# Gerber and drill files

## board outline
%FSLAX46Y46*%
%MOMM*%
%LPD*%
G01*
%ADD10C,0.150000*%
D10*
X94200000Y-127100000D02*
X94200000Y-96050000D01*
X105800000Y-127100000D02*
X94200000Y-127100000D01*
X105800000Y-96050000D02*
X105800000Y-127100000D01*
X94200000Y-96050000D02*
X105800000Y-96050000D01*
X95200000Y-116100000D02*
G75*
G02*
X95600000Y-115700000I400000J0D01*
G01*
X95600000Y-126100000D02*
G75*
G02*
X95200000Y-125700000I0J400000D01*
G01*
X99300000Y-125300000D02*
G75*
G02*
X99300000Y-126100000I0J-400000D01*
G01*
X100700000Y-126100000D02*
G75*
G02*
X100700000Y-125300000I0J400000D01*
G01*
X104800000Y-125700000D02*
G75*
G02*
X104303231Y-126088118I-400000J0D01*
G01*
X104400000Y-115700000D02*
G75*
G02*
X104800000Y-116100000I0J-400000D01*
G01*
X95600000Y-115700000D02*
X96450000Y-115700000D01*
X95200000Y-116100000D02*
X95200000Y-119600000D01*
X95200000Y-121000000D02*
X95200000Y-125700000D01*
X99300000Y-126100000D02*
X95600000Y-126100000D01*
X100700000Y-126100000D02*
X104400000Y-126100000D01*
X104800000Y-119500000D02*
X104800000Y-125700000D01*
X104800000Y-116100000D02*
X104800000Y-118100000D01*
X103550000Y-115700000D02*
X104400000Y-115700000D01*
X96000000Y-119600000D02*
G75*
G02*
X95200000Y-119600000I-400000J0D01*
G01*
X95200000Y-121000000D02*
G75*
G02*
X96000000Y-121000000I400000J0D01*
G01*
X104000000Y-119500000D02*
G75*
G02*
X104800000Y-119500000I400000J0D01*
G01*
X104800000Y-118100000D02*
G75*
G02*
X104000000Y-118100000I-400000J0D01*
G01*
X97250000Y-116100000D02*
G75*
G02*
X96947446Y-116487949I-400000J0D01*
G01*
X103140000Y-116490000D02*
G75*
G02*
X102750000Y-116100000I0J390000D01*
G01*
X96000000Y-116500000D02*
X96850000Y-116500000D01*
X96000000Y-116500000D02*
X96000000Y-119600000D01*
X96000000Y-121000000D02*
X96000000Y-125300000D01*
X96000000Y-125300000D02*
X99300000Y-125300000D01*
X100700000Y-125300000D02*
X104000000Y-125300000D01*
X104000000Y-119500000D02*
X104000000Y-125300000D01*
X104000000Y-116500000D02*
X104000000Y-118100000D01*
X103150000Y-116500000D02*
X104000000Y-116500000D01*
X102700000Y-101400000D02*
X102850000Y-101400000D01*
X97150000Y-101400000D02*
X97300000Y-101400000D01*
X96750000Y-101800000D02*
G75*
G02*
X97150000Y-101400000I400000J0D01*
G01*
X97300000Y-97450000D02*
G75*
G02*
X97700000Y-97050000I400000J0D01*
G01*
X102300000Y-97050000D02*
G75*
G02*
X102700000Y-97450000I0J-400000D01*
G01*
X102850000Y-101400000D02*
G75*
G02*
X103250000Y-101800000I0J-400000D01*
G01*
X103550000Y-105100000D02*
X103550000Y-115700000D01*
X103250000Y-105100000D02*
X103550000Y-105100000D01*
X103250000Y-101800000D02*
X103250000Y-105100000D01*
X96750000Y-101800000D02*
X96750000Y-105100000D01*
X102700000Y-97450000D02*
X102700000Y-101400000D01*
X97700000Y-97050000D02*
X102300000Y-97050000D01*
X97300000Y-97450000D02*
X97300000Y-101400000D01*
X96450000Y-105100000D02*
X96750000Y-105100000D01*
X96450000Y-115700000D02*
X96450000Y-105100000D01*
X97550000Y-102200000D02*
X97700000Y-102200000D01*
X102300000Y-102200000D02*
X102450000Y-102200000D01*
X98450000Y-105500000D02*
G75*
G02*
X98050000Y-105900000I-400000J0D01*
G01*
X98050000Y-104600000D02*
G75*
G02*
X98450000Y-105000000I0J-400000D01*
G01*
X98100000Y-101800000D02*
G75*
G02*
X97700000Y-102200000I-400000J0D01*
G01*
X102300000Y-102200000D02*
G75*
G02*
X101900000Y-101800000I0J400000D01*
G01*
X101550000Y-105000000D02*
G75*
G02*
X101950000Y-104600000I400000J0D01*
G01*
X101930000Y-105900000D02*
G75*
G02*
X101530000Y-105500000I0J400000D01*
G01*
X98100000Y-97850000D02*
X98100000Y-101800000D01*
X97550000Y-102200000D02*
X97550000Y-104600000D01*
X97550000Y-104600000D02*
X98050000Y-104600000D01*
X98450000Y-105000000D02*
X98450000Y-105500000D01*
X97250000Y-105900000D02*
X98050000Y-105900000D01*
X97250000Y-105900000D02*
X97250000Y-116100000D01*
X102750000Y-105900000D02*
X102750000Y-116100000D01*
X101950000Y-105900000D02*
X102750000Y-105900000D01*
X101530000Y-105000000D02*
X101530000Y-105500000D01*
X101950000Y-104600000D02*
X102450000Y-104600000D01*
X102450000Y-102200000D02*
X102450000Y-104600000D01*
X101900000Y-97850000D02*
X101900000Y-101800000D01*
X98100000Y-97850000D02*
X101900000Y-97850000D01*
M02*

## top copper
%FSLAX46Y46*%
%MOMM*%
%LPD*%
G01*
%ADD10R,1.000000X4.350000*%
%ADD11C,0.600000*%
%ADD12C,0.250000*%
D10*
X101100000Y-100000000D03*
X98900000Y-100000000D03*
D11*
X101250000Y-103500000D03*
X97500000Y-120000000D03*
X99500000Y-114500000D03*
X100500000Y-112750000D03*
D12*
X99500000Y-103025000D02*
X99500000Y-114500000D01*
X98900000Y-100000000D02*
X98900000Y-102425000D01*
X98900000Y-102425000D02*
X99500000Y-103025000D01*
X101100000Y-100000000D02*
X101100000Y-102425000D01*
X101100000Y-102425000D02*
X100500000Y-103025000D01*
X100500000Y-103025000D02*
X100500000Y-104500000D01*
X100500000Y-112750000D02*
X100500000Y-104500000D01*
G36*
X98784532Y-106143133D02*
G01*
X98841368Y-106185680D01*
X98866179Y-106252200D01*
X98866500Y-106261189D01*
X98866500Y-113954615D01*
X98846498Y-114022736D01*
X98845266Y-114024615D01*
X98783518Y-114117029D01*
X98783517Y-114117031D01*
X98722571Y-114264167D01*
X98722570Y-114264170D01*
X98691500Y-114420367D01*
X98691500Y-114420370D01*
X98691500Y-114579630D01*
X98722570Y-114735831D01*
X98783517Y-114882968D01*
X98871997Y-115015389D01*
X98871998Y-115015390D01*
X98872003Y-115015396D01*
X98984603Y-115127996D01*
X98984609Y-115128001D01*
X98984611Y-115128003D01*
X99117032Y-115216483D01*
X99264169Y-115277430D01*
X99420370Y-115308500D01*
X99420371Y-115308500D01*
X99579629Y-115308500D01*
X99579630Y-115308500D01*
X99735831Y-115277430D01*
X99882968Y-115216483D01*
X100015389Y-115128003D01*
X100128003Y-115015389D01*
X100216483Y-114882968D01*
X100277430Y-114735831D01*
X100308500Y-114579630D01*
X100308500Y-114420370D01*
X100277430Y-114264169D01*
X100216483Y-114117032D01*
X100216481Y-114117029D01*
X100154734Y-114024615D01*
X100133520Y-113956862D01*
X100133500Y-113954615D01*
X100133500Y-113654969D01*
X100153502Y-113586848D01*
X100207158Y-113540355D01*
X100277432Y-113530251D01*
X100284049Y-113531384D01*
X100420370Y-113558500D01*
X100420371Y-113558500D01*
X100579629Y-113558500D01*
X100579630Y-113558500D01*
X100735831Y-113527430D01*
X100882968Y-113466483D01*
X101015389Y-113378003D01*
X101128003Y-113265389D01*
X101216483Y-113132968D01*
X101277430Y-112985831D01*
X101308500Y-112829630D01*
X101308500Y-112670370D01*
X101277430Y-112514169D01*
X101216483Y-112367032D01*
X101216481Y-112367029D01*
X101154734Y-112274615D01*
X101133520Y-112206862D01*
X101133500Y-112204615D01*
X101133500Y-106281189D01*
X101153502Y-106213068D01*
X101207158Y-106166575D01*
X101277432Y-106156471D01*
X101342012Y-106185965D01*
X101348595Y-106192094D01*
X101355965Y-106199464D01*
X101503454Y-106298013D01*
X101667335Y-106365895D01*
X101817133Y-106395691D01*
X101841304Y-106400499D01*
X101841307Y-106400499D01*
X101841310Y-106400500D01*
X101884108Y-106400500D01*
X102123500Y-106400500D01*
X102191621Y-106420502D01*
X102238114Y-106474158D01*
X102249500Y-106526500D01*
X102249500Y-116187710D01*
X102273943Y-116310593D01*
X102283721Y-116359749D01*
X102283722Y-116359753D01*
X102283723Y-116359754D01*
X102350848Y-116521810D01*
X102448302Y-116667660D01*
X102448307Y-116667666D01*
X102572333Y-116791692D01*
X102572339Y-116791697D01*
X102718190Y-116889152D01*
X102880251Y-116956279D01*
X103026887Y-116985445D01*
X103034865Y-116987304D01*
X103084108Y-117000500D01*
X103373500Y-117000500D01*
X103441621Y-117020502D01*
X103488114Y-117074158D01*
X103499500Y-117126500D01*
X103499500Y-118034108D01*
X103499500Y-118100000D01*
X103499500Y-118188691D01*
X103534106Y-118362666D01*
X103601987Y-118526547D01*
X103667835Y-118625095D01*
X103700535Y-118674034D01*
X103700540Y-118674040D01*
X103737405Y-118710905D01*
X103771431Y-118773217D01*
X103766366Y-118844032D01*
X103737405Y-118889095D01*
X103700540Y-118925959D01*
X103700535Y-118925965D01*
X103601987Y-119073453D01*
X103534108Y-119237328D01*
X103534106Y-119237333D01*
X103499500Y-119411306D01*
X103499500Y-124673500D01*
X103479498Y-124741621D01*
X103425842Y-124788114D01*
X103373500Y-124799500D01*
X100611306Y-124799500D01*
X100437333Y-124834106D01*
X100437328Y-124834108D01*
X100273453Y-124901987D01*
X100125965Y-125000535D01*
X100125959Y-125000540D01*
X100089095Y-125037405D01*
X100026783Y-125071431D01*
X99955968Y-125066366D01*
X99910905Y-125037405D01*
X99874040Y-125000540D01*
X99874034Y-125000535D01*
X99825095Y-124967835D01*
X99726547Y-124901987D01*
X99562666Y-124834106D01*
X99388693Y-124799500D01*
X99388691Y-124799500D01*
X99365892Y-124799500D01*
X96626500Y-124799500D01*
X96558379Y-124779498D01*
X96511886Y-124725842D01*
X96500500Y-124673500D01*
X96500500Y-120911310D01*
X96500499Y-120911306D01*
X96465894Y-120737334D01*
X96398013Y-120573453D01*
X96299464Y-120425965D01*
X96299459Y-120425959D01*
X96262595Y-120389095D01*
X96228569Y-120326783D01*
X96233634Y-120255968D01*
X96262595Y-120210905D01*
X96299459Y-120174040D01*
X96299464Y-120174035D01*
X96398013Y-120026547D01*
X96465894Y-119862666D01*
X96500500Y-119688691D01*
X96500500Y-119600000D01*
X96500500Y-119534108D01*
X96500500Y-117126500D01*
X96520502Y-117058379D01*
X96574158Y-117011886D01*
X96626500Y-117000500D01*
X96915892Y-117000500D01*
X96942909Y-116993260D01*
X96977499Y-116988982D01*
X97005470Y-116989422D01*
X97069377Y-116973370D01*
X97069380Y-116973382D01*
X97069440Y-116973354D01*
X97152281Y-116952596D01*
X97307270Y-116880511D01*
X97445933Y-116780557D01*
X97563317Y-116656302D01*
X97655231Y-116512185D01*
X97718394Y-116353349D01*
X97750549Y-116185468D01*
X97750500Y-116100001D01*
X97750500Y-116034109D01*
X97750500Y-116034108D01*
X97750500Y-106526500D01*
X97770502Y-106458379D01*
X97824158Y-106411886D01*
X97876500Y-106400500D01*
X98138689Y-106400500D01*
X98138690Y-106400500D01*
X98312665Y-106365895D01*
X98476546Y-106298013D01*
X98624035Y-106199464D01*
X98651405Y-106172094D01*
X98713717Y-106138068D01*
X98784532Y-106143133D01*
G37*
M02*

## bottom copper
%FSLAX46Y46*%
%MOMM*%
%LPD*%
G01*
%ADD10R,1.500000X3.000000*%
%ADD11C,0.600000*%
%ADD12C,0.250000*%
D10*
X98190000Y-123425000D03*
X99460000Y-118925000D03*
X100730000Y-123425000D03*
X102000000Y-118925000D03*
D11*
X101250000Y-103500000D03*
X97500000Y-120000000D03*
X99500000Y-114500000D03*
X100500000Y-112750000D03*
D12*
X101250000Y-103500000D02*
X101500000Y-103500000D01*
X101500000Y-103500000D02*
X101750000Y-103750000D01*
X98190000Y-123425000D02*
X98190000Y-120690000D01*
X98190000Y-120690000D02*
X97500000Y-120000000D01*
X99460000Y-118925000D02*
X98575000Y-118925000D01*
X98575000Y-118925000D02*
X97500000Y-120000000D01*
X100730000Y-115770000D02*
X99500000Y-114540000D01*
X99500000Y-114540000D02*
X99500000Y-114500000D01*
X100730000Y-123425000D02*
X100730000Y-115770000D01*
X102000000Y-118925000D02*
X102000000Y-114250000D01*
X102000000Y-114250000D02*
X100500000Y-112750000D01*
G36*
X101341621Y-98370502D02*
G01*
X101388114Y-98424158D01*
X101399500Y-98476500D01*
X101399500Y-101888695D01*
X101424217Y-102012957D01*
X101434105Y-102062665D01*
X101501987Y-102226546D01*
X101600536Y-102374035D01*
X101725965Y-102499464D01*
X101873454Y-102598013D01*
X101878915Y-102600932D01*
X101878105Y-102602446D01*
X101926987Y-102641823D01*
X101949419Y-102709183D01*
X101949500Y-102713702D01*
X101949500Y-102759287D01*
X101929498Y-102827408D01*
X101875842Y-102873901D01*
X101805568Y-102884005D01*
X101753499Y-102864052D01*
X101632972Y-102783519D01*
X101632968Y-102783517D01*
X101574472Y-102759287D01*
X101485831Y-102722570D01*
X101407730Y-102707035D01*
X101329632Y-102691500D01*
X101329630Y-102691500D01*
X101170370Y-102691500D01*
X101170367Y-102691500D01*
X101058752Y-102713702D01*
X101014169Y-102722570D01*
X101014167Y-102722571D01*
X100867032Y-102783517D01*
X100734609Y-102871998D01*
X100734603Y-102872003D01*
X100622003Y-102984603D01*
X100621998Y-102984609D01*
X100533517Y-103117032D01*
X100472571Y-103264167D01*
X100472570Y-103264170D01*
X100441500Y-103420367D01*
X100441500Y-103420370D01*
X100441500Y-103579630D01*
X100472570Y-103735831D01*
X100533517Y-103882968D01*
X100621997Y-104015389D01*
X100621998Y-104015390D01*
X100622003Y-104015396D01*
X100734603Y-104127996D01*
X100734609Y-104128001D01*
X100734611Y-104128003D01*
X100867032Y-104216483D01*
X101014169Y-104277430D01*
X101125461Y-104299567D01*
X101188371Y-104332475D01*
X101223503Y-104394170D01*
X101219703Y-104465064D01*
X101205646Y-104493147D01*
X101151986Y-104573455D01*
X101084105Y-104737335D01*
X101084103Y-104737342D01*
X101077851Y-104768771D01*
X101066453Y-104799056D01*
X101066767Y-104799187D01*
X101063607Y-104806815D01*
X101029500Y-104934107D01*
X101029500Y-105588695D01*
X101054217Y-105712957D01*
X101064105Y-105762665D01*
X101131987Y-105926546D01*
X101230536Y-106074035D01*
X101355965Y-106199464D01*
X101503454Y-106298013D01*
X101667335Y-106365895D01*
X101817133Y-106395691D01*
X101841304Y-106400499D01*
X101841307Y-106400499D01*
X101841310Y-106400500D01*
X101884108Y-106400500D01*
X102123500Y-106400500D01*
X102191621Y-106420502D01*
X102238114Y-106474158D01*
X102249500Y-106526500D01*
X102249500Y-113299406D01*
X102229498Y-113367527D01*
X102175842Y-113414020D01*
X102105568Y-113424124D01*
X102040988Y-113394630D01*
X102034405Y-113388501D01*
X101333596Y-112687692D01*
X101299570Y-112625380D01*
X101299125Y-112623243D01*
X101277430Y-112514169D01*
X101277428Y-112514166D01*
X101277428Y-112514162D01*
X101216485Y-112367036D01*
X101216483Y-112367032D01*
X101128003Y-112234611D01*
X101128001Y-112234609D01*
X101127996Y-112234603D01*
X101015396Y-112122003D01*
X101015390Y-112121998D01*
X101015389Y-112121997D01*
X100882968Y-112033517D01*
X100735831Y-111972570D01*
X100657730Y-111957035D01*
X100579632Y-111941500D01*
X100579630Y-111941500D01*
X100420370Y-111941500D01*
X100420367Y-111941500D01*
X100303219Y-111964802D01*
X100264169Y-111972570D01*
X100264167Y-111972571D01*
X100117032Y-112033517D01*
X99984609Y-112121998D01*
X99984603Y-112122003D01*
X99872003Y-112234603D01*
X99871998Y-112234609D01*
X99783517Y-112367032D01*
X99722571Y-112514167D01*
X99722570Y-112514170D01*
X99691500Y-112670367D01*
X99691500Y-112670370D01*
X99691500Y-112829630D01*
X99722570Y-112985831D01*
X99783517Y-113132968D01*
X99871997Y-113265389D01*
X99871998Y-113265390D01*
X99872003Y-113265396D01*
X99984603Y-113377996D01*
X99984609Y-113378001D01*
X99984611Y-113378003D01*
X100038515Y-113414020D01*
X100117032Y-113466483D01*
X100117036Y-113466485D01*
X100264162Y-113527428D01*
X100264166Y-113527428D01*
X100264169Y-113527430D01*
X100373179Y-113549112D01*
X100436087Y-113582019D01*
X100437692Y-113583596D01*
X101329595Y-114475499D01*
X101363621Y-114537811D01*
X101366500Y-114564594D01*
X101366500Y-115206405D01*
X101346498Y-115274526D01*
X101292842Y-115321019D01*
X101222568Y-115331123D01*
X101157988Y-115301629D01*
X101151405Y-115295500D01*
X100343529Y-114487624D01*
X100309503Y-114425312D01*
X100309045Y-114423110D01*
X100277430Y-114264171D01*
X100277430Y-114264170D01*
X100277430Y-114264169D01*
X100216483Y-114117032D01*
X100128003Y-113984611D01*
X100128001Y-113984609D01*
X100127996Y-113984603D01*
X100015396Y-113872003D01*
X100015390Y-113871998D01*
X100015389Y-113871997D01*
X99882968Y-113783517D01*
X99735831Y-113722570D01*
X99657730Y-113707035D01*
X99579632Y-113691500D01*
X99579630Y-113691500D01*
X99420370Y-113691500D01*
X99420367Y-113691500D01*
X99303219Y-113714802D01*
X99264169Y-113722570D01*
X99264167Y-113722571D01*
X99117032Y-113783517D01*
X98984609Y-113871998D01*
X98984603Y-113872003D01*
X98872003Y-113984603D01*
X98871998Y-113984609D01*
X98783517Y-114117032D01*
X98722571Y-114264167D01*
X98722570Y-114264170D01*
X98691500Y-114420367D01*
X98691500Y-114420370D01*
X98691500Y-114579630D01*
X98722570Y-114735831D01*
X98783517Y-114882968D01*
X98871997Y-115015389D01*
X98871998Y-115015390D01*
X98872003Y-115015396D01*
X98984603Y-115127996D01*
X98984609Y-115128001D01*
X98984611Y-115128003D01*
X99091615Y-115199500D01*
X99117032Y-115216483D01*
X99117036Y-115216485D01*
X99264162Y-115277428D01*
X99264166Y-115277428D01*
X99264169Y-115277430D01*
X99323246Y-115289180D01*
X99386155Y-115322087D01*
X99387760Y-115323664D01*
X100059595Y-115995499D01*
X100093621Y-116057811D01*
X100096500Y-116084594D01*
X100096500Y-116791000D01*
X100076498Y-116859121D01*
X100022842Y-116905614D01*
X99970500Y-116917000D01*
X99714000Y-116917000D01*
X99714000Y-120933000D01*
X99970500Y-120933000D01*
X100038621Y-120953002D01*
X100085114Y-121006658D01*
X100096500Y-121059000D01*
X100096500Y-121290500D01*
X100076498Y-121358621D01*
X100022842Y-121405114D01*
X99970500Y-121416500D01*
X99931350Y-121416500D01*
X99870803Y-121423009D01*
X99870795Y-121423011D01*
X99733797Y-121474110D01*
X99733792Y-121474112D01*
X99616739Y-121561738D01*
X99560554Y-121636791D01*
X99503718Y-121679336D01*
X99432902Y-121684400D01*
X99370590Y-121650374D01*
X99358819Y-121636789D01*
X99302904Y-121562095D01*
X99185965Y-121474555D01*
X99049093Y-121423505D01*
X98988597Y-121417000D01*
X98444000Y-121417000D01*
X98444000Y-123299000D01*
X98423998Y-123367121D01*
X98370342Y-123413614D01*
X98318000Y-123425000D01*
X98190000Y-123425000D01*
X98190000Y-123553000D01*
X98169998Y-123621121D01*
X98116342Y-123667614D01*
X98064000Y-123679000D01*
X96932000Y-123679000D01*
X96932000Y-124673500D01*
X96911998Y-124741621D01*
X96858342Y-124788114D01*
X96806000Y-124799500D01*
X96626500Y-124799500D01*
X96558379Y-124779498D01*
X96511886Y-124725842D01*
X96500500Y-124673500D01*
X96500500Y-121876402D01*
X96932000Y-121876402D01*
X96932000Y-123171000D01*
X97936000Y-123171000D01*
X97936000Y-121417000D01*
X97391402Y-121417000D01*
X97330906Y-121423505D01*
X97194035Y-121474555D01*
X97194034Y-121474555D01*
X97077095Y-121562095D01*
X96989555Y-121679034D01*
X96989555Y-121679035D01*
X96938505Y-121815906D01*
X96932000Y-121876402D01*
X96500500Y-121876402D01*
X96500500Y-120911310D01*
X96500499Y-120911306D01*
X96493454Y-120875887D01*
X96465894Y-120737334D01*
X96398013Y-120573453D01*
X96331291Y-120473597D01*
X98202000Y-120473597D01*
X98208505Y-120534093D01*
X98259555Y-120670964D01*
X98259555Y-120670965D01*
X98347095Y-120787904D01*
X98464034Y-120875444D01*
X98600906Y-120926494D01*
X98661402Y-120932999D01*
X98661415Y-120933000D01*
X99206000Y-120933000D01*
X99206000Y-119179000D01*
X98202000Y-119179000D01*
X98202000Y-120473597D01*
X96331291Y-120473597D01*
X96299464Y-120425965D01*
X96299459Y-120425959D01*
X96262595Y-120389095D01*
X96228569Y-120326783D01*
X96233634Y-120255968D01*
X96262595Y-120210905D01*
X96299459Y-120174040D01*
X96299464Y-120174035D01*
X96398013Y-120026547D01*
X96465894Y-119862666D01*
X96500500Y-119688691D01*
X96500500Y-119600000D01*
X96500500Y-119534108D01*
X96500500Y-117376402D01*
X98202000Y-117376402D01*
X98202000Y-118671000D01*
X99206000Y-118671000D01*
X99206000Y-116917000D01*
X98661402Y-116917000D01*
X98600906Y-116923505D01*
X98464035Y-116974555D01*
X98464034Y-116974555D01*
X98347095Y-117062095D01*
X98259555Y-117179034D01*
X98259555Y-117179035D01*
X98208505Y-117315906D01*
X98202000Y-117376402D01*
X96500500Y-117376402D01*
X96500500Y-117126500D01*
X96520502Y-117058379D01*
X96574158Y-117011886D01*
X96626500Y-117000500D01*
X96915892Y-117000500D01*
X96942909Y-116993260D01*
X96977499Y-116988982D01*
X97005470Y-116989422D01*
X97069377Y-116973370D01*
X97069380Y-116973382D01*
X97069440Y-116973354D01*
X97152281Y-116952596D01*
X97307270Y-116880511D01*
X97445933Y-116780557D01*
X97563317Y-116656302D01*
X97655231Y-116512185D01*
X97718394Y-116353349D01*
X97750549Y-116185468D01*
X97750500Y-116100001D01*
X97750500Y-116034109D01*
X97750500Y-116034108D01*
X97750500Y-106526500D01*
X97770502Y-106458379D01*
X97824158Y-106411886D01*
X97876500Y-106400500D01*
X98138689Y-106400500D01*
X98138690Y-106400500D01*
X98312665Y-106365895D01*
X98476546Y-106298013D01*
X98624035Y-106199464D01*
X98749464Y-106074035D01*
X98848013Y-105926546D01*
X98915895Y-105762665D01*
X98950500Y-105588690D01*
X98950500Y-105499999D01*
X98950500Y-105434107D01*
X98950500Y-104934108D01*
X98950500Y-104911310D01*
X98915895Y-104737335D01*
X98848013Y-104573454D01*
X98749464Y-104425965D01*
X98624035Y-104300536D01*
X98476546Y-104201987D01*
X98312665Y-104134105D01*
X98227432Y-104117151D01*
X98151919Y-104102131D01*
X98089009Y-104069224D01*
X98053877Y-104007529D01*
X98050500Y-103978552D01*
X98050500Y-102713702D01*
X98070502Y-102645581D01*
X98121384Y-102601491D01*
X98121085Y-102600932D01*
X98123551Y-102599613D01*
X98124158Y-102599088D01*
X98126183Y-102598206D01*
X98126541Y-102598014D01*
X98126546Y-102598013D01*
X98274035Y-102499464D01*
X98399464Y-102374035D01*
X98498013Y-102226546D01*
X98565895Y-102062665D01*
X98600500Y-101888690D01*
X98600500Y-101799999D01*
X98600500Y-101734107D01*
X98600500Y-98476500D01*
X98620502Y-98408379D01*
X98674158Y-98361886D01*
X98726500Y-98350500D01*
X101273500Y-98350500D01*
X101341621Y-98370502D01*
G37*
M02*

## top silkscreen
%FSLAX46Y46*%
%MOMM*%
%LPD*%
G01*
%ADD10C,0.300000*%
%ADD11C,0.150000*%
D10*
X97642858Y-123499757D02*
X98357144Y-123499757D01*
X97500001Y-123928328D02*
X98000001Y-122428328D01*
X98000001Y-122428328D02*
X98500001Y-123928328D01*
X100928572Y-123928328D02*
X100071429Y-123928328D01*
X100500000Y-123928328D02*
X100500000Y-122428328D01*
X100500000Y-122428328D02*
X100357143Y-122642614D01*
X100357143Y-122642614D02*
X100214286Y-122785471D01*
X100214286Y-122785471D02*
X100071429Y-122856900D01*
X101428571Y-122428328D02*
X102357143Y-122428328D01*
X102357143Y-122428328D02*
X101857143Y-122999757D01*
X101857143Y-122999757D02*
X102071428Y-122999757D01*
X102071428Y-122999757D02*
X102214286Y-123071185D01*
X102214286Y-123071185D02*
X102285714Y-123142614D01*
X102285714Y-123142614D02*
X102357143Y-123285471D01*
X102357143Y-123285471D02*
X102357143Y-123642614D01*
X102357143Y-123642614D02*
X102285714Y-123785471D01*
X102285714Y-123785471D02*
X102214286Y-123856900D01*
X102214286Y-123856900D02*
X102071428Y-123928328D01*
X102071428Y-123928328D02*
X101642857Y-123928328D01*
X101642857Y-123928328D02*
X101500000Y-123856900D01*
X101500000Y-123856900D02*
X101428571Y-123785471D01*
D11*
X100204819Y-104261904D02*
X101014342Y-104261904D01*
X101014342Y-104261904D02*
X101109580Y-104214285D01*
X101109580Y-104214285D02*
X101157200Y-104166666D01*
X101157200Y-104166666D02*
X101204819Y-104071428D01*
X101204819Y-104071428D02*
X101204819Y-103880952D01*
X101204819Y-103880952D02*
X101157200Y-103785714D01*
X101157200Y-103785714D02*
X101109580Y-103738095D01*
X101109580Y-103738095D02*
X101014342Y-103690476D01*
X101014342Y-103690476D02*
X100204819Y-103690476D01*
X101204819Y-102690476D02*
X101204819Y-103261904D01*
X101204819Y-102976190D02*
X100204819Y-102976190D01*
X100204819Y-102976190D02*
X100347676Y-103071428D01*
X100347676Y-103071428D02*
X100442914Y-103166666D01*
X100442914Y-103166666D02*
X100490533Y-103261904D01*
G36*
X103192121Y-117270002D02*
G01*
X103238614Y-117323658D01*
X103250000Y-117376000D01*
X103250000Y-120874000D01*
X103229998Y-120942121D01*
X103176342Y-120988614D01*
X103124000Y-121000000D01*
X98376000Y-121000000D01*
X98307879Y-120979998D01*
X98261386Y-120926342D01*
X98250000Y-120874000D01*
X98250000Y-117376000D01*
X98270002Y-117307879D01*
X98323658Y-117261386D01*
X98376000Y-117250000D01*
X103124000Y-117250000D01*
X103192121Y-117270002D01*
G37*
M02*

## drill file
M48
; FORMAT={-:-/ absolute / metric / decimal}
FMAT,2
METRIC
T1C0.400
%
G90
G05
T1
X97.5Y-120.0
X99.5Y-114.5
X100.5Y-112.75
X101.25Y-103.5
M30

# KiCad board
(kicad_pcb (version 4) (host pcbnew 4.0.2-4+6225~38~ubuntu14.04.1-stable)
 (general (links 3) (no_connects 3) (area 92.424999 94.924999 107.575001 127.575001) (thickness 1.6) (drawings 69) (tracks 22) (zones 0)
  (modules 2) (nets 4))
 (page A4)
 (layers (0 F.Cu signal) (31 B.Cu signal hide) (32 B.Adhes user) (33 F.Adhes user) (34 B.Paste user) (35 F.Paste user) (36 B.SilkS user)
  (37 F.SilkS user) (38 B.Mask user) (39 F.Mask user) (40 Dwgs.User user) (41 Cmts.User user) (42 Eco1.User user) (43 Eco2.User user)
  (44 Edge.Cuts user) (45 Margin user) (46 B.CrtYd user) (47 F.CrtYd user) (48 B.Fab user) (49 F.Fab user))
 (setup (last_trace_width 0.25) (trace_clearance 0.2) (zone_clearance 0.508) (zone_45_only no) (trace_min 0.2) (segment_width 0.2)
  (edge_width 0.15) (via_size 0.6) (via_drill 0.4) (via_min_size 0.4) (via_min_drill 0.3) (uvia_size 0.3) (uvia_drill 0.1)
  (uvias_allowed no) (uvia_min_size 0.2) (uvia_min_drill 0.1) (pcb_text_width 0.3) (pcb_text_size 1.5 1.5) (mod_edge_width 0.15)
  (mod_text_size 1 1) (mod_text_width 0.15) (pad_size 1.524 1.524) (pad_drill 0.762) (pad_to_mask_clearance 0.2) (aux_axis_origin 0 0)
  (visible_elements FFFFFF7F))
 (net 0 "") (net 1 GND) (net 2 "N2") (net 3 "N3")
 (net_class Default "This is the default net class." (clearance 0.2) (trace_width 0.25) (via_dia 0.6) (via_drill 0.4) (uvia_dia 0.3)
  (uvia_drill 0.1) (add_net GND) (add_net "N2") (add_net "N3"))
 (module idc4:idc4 (layer B.Cu) (at 100.095 121.175 180)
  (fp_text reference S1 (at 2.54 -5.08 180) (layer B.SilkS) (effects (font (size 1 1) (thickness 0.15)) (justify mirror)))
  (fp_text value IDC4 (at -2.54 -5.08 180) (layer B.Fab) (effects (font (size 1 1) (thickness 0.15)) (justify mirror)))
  (pad 1 smd rect (at 1.905 -2.25 180) (size 1.5 3) (layers B.Cu B.Paste B.Mask) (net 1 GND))
  (pad 2 smd rect (at 0.635 2.25 180) (size 1.5 3) (layers B.Cu B.Paste B.Mask) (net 1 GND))
  (pad 3 smd rect (at -0.635 -2.25 180) (size 1.5 3) (layers B.Cu B.Paste B.Mask) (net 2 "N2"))
  (pad 4 smd rect (at -1.905 2.25 180) (size 1.5 3) (layers B.Cu B.Paste B.Mask) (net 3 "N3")))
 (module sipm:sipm (layer F.Cu) (at 100 100)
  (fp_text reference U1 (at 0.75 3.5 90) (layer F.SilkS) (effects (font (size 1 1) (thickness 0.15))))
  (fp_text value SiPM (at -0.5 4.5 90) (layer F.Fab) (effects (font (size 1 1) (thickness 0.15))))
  (pad 1 smd rect (at 1.1 0) (size 1 4.35) (layers F.Cu F.Paste F.Mask) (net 3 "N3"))
  (pad 2 smd rect (at -1.1 0) (size 1 4.35) (layers F.Cu F.Paste F.Mask) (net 2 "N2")))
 (gr_line (start 94.2 127.1) (end 94.2 96.05) (layer Edge.Cuts) (width 0.15))
 (gr_line (start 105.8 127.1) (end 94.2 127.1) (layer Edge.Cuts) (width 0.15))
 (gr_line (start 105.8 96.05) (end 105.8 127.1) (layer Edge.Cuts) (width 0.15))
 (gr_line (start 94.2 96.05) (end 105.8 96.05) (layer Edge.Cuts) (width 0.15))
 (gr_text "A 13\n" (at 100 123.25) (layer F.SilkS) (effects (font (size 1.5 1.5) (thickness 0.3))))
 (gr_arc (start 95.6 116.1) (end 95.6 115.7) (angle -90) (layer Edge.Cuts) (width 0.15))
 (gr_arc (start 95.6 125.7) (end 95.2 125.7) (angle -90) (layer Edge.Cuts) (width 0.15))
 (gr_arc (start 99.3 125.7) (end 99.3 125.3) (angle 180) (layer Edge.Cuts) (width 0.15))
 (gr_arc (start 100.7 125.7) (end 100.7 125.3) (angle -180) (layer Edge.Cuts) (width 0.15))
 (gr_arc (start 104.4 125.7) (end 104.8 125.7) (angle 104) (layer Edge.Cuts) (width 0.15))
 (gr_arc (start 104.4 116.1) (end 104.8 116.1) (angle -90) (layer Edge.Cuts) (width 0.15))
 (gr_line (start 95.6 115.7) (end 96.45 115.7) (layer Edge.Cuts) (width 0.15))
 (gr_line (start 95.2 116.1) (end 95.2 119.6) (layer Edge.Cuts) (width 0.15))
 (gr_line (start 95.2 121) (end 95.2 125.7) (layer Edge.Cuts) (width 0.15))
 (gr_line (start 99.3 126.1) (end 95.6 126.1) (layer Edge.Cuts) (width 0.15))
 (gr_line (start 100.7 126.1) (end 104.4 126.1) (layer Edge.Cuts) (width 0.15))
 (gr_line (start 104.8 119.5) (end 104.8 125.7) (layer Edge.Cuts) (width 0.15))
 (gr_line (start 104.8 116.1) (end 104.8 118.1) (layer Edge.Cuts) (width 0.15))
 (gr_line (start 103.55 115.7) (end 104.4 115.7) (layer Edge.Cuts) (width 0.15))
 (gr_arc (start 95.6 119.6) (end 96 119.6) (angle 180) (layer Edge.Cuts) (width 0.15))
 (gr_arc (start 95.6 121) (end 96 121) (angle -180) (layer Edge.Cuts) (width 0.15))
 (gr_arc (start 104.4 119.5) (end 104 119.5) (angle 180) (layer Edge.Cuts) (width 0.15))
 (gr_arc (start 104.4 118.1) (end 104 118.1) (angle -180) (layer Edge.Cuts) (width 0.15))
 (gr_arc (start 96.85 116.1) (end 97.25 116.1) (angle 75.9) (layer Edge.Cuts) (width 0.15))
 (gr_arc (start 103.14 116.1) (end 102.75 116.1) (angle -90) (layer Edge.Cuts) (width 0.15))
 (gr_line (start 96 116.5) (end 96.85 116.5) (layer Edge.Cuts) (width 0.15))
 (gr_line (start 96 116.5) (end 96 119.6) (layer Edge.Cuts) (width 0.15))
 (gr_line (start 96 121) (end 96 125.3) (layer Edge.Cuts) (width 0.15))
 (gr_line (start 96 125.3) (end 99.3 125.3) (layer Edge.Cuts) (width 0.15))
 (gr_line (start 100.7 125.3) (end 104 125.3) (layer Edge.Cuts) (width 0.15))
 (gr_line (start 104 119.5) (end 104 125.3) (layer Edge.Cuts) (width 0.15))
 (gr_line (start 104 116.5) (end 104 118.1) (layer Edge.Cuts) (width 0.15))
 (gr_line (start 103.15 116.5) (end 104 116.5) (layer Edge.Cuts) (width 0.15))
 (gr_line (start 102.7 101.4) (end 102.85 101.4) (layer Edge.Cuts) (width 0.15))
 (gr_line (start 97.15 101.4) (end 97.3 101.4) (layer Edge.Cuts) (width 0.15))
 (gr_arc (start 97.15 101.8) (end 97.15 101.4) (angle -90) (layer Edge.Cuts) (width 0.15))
 (gr_arc (start 97.7 97.45) (end 97.3 97.45) (angle 90) (layer Edge.Cuts) (width 0.15))
 (gr_arc (start 102.3 97.45) (end 102.3 97.05) (angle 90) (layer Edge.Cuts) (width 0.15))
 (gr_arc (start 102.85 101.8) (end 102.85 101.4) (angle 90) (layer Edge.Cuts) (width 0.15))
 (gr_line (start 103.55 105.1) (end 103.55 115.7) (layer Edge.Cuts) (width 0.15))
 (gr_line (start 103.25 105.1) (end 103.55 105.1) (layer Edge.Cuts) (width 0.15))
 (gr_line (start 103.25 101.8) (end 103.25 105.1) (layer Edge.Cuts) (width 0.15))
 (gr_line (start 96.75 101.8) (end 96.75 105.1) (layer Edge.Cuts) (width 0.15))
 (gr_line (start 102.7 97.45) (end 102.7 101.4) (layer Edge.Cuts) (width 0.15))
 (gr_line (start 97.7 97.05) (end 102.3 97.05) (layer Edge.Cuts) (width 0.15))
 (gr_line (start 97.3 97.45) (end 97.3 101.4) (layer Edge.Cuts) (width 0.15))
 (gr_line (start 96.45 105.1) (end 96.75 105.1) (layer Edge.Cuts) (width 0.15))
 (gr_line (start 96.45 115.7) (end 96.45 105.1) (layer Edge.Cuts) (width 0.15))
 (gr_line (start 97.55 102.2) (end 97.7 102.2) (layer Edge.Cuts) (width 0.15))
 (gr_line (start 102.3 102.2) (end 102.45 102.2) (layer Edge.Cuts) (width 0.15))
 (gr_arc (start 98.05 105.5) (end 98.05 105.9) (angle -90) (layer Edge.Cuts) (width 0.15))
 (gr_arc (start 98.05 105) (end 98.05 104.6) (angle 90) (layer Edge.Cuts) (width 0.15))
 (gr_arc (start 97.7 101.8) (end 97.7 102.2) (angle -90) (layer Edge.Cuts) (width 0.15))
 (gr_arc (start 102.3 101.8) (end 101.9 101.8) (angle -90) (layer Edge.Cuts) (width 0.15))
 (gr_arc (start 101.95 105) (end 101.95 104.6) (angle -90) (layer Edge.Cuts) (width 0.15))
 (gr_arc (start 101.93 105.5) (end 101.53 105.5) (angle -90) (layer Edge.Cuts) (width 0.15))
 (gr_line (start 98.1 97.85) (end 98.1 101.8) (layer Edge.Cuts) (width 0.15))
 (gr_line (start 97.55 102.2) (end 97.55 104.6) (layer Edge.Cuts) (width 0.15))
 (gr_line (start 97.55 104.6) (end 98.05 104.6) (layer Edge.Cuts) (width 0.15))
 (gr_line (start 98.45 105) (end 98.45 105.5) (layer Edge.Cuts) (width 0.15))
 (gr_line (start 97.25 105.9) (end 98.05 105.9) (layer Edge.Cuts) (width 0.15))
 (gr_line (start 97.25 105.9) (end 97.25 116.1) (layer Edge.Cuts) (width 0.15))
 (gr_line (start 102.75 105.9) (end 102.75 116.1) (layer Edge.Cuts) (width 0.15))
 (gr_line (start 101.95 105.9) (end 102.75 105.9) (layer Edge.Cuts) (width 0.15))
 (gr_line (start 101.53 105) (end 101.53 105.5) (layer Edge.Cuts) (width 0.15))
 (gr_line (start 101.95 104.6) (end 102.45 104.6) (layer Edge.Cuts) (width 0.15))
 (gr_line (start 102.45 102.2) (end 102.45 104.6) (layer Edge.Cuts) (width 0.15))
 (gr_line (start 101.9 97.85) (end 101.9 101.8) (layer Edge.Cuts) (width 0.15))
 (gr_line (start 98.1 97.85) (end 101.9 97.85) (layer Edge.Cuts) (width 0.15))
 (segment (start 101.25 103.5) (end 101.5 103.5) (width 0.25) (layer B.Cu) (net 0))
 (segment (start 101.5 103.5) (end 101.75 103.75) (width 0.25) (layer B.Cu) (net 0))
 (via (at 101.25 103.5) (size 0.6) (drill 0.4) (layers F.Cu B.Cu) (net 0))
 (segment (start 98.19 123.425) (end 98.19 120.69) (width 0.25) (layer B.Cu) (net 1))
 (segment (start 98.19 120.69) (end 97.5 120) (width 0.25) (layer B.Cu) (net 1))
 (segment (start 99.46 118.925) (end 98.575 118.925) (width 0.25) (layer B.Cu) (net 1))
 (segment (start 98.575 118.925) (end 97.5 120) (width 0.25) (layer B.Cu) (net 1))
 (via (at 97.5 120) (size 0.6) (drill 0.4) (layers F.Cu B.Cu) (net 1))
 (segment (start 99.5 103.025) (end 99.5 114.5) (width 0.25) (layer F.Cu) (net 2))
 (segment (start 98.9 100) (end 98.9 102.425) (width 0.25) (layer F.Cu) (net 2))
 (segment (start 98.9 102.425) (end 99.5 103.025) (width 0.25) (layer F.Cu) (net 2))
 (segment (start 100.73 115.77) (end 99.5 114.54) (width 0.25) (layer B.Cu) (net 2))
 (segment (start 99.5 114.54) (end 99.5 114.5) (width 0.25) (layer B.Cu) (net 2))
 (via (at 99.5 114.5) (size 0.6) (drill 0.4) (layers F.Cu B.Cu) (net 2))
 (segment (start 100.73 123.425) (end 100.73 115.77) (width 0.25) (layer B.Cu) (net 2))
 (segment (start 101.1 100) (end 101.1 102.425) (width 0.25) (layer F.Cu) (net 3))
 (segment (start 101.1 102.425) (end 100.5 103.025) (width 0.25) (layer F.Cu) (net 3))
 (segment (start 100.5 103.025) (end 100.5 104.5) (width 0.25) (layer F.Cu) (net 3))
 (segment (start 100.5 112.75) (end 100.5 104.5) (width 0.25) (layer F.Cu) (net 3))
 (segment (start 102 118.925) (end 102 114.25) (width 0.25) (layer B.Cu) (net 3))
 (segment (start 102 114.25) (end 100.5 112.75) (width 0.25) (layer B.Cu) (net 3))
 (via (at 100.5 112.75) (size 0.6) (drill 0.4) (layers F.Cu B.Cu) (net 3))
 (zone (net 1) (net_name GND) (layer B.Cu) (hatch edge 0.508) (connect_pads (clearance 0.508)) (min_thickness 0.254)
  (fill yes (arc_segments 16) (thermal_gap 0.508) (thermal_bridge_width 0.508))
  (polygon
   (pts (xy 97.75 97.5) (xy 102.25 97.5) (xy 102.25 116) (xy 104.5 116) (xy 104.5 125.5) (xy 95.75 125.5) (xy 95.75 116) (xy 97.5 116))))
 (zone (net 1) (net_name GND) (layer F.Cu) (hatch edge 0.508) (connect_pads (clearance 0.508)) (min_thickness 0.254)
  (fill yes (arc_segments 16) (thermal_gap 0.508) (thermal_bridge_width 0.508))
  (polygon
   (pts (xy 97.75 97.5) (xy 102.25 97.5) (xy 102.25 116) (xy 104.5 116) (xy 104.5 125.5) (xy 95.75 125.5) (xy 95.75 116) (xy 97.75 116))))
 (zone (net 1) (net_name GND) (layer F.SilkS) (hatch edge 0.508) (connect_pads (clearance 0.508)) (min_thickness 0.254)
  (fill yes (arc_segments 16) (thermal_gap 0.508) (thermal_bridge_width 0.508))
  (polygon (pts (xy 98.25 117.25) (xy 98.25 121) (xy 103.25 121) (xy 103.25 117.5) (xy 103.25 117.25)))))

